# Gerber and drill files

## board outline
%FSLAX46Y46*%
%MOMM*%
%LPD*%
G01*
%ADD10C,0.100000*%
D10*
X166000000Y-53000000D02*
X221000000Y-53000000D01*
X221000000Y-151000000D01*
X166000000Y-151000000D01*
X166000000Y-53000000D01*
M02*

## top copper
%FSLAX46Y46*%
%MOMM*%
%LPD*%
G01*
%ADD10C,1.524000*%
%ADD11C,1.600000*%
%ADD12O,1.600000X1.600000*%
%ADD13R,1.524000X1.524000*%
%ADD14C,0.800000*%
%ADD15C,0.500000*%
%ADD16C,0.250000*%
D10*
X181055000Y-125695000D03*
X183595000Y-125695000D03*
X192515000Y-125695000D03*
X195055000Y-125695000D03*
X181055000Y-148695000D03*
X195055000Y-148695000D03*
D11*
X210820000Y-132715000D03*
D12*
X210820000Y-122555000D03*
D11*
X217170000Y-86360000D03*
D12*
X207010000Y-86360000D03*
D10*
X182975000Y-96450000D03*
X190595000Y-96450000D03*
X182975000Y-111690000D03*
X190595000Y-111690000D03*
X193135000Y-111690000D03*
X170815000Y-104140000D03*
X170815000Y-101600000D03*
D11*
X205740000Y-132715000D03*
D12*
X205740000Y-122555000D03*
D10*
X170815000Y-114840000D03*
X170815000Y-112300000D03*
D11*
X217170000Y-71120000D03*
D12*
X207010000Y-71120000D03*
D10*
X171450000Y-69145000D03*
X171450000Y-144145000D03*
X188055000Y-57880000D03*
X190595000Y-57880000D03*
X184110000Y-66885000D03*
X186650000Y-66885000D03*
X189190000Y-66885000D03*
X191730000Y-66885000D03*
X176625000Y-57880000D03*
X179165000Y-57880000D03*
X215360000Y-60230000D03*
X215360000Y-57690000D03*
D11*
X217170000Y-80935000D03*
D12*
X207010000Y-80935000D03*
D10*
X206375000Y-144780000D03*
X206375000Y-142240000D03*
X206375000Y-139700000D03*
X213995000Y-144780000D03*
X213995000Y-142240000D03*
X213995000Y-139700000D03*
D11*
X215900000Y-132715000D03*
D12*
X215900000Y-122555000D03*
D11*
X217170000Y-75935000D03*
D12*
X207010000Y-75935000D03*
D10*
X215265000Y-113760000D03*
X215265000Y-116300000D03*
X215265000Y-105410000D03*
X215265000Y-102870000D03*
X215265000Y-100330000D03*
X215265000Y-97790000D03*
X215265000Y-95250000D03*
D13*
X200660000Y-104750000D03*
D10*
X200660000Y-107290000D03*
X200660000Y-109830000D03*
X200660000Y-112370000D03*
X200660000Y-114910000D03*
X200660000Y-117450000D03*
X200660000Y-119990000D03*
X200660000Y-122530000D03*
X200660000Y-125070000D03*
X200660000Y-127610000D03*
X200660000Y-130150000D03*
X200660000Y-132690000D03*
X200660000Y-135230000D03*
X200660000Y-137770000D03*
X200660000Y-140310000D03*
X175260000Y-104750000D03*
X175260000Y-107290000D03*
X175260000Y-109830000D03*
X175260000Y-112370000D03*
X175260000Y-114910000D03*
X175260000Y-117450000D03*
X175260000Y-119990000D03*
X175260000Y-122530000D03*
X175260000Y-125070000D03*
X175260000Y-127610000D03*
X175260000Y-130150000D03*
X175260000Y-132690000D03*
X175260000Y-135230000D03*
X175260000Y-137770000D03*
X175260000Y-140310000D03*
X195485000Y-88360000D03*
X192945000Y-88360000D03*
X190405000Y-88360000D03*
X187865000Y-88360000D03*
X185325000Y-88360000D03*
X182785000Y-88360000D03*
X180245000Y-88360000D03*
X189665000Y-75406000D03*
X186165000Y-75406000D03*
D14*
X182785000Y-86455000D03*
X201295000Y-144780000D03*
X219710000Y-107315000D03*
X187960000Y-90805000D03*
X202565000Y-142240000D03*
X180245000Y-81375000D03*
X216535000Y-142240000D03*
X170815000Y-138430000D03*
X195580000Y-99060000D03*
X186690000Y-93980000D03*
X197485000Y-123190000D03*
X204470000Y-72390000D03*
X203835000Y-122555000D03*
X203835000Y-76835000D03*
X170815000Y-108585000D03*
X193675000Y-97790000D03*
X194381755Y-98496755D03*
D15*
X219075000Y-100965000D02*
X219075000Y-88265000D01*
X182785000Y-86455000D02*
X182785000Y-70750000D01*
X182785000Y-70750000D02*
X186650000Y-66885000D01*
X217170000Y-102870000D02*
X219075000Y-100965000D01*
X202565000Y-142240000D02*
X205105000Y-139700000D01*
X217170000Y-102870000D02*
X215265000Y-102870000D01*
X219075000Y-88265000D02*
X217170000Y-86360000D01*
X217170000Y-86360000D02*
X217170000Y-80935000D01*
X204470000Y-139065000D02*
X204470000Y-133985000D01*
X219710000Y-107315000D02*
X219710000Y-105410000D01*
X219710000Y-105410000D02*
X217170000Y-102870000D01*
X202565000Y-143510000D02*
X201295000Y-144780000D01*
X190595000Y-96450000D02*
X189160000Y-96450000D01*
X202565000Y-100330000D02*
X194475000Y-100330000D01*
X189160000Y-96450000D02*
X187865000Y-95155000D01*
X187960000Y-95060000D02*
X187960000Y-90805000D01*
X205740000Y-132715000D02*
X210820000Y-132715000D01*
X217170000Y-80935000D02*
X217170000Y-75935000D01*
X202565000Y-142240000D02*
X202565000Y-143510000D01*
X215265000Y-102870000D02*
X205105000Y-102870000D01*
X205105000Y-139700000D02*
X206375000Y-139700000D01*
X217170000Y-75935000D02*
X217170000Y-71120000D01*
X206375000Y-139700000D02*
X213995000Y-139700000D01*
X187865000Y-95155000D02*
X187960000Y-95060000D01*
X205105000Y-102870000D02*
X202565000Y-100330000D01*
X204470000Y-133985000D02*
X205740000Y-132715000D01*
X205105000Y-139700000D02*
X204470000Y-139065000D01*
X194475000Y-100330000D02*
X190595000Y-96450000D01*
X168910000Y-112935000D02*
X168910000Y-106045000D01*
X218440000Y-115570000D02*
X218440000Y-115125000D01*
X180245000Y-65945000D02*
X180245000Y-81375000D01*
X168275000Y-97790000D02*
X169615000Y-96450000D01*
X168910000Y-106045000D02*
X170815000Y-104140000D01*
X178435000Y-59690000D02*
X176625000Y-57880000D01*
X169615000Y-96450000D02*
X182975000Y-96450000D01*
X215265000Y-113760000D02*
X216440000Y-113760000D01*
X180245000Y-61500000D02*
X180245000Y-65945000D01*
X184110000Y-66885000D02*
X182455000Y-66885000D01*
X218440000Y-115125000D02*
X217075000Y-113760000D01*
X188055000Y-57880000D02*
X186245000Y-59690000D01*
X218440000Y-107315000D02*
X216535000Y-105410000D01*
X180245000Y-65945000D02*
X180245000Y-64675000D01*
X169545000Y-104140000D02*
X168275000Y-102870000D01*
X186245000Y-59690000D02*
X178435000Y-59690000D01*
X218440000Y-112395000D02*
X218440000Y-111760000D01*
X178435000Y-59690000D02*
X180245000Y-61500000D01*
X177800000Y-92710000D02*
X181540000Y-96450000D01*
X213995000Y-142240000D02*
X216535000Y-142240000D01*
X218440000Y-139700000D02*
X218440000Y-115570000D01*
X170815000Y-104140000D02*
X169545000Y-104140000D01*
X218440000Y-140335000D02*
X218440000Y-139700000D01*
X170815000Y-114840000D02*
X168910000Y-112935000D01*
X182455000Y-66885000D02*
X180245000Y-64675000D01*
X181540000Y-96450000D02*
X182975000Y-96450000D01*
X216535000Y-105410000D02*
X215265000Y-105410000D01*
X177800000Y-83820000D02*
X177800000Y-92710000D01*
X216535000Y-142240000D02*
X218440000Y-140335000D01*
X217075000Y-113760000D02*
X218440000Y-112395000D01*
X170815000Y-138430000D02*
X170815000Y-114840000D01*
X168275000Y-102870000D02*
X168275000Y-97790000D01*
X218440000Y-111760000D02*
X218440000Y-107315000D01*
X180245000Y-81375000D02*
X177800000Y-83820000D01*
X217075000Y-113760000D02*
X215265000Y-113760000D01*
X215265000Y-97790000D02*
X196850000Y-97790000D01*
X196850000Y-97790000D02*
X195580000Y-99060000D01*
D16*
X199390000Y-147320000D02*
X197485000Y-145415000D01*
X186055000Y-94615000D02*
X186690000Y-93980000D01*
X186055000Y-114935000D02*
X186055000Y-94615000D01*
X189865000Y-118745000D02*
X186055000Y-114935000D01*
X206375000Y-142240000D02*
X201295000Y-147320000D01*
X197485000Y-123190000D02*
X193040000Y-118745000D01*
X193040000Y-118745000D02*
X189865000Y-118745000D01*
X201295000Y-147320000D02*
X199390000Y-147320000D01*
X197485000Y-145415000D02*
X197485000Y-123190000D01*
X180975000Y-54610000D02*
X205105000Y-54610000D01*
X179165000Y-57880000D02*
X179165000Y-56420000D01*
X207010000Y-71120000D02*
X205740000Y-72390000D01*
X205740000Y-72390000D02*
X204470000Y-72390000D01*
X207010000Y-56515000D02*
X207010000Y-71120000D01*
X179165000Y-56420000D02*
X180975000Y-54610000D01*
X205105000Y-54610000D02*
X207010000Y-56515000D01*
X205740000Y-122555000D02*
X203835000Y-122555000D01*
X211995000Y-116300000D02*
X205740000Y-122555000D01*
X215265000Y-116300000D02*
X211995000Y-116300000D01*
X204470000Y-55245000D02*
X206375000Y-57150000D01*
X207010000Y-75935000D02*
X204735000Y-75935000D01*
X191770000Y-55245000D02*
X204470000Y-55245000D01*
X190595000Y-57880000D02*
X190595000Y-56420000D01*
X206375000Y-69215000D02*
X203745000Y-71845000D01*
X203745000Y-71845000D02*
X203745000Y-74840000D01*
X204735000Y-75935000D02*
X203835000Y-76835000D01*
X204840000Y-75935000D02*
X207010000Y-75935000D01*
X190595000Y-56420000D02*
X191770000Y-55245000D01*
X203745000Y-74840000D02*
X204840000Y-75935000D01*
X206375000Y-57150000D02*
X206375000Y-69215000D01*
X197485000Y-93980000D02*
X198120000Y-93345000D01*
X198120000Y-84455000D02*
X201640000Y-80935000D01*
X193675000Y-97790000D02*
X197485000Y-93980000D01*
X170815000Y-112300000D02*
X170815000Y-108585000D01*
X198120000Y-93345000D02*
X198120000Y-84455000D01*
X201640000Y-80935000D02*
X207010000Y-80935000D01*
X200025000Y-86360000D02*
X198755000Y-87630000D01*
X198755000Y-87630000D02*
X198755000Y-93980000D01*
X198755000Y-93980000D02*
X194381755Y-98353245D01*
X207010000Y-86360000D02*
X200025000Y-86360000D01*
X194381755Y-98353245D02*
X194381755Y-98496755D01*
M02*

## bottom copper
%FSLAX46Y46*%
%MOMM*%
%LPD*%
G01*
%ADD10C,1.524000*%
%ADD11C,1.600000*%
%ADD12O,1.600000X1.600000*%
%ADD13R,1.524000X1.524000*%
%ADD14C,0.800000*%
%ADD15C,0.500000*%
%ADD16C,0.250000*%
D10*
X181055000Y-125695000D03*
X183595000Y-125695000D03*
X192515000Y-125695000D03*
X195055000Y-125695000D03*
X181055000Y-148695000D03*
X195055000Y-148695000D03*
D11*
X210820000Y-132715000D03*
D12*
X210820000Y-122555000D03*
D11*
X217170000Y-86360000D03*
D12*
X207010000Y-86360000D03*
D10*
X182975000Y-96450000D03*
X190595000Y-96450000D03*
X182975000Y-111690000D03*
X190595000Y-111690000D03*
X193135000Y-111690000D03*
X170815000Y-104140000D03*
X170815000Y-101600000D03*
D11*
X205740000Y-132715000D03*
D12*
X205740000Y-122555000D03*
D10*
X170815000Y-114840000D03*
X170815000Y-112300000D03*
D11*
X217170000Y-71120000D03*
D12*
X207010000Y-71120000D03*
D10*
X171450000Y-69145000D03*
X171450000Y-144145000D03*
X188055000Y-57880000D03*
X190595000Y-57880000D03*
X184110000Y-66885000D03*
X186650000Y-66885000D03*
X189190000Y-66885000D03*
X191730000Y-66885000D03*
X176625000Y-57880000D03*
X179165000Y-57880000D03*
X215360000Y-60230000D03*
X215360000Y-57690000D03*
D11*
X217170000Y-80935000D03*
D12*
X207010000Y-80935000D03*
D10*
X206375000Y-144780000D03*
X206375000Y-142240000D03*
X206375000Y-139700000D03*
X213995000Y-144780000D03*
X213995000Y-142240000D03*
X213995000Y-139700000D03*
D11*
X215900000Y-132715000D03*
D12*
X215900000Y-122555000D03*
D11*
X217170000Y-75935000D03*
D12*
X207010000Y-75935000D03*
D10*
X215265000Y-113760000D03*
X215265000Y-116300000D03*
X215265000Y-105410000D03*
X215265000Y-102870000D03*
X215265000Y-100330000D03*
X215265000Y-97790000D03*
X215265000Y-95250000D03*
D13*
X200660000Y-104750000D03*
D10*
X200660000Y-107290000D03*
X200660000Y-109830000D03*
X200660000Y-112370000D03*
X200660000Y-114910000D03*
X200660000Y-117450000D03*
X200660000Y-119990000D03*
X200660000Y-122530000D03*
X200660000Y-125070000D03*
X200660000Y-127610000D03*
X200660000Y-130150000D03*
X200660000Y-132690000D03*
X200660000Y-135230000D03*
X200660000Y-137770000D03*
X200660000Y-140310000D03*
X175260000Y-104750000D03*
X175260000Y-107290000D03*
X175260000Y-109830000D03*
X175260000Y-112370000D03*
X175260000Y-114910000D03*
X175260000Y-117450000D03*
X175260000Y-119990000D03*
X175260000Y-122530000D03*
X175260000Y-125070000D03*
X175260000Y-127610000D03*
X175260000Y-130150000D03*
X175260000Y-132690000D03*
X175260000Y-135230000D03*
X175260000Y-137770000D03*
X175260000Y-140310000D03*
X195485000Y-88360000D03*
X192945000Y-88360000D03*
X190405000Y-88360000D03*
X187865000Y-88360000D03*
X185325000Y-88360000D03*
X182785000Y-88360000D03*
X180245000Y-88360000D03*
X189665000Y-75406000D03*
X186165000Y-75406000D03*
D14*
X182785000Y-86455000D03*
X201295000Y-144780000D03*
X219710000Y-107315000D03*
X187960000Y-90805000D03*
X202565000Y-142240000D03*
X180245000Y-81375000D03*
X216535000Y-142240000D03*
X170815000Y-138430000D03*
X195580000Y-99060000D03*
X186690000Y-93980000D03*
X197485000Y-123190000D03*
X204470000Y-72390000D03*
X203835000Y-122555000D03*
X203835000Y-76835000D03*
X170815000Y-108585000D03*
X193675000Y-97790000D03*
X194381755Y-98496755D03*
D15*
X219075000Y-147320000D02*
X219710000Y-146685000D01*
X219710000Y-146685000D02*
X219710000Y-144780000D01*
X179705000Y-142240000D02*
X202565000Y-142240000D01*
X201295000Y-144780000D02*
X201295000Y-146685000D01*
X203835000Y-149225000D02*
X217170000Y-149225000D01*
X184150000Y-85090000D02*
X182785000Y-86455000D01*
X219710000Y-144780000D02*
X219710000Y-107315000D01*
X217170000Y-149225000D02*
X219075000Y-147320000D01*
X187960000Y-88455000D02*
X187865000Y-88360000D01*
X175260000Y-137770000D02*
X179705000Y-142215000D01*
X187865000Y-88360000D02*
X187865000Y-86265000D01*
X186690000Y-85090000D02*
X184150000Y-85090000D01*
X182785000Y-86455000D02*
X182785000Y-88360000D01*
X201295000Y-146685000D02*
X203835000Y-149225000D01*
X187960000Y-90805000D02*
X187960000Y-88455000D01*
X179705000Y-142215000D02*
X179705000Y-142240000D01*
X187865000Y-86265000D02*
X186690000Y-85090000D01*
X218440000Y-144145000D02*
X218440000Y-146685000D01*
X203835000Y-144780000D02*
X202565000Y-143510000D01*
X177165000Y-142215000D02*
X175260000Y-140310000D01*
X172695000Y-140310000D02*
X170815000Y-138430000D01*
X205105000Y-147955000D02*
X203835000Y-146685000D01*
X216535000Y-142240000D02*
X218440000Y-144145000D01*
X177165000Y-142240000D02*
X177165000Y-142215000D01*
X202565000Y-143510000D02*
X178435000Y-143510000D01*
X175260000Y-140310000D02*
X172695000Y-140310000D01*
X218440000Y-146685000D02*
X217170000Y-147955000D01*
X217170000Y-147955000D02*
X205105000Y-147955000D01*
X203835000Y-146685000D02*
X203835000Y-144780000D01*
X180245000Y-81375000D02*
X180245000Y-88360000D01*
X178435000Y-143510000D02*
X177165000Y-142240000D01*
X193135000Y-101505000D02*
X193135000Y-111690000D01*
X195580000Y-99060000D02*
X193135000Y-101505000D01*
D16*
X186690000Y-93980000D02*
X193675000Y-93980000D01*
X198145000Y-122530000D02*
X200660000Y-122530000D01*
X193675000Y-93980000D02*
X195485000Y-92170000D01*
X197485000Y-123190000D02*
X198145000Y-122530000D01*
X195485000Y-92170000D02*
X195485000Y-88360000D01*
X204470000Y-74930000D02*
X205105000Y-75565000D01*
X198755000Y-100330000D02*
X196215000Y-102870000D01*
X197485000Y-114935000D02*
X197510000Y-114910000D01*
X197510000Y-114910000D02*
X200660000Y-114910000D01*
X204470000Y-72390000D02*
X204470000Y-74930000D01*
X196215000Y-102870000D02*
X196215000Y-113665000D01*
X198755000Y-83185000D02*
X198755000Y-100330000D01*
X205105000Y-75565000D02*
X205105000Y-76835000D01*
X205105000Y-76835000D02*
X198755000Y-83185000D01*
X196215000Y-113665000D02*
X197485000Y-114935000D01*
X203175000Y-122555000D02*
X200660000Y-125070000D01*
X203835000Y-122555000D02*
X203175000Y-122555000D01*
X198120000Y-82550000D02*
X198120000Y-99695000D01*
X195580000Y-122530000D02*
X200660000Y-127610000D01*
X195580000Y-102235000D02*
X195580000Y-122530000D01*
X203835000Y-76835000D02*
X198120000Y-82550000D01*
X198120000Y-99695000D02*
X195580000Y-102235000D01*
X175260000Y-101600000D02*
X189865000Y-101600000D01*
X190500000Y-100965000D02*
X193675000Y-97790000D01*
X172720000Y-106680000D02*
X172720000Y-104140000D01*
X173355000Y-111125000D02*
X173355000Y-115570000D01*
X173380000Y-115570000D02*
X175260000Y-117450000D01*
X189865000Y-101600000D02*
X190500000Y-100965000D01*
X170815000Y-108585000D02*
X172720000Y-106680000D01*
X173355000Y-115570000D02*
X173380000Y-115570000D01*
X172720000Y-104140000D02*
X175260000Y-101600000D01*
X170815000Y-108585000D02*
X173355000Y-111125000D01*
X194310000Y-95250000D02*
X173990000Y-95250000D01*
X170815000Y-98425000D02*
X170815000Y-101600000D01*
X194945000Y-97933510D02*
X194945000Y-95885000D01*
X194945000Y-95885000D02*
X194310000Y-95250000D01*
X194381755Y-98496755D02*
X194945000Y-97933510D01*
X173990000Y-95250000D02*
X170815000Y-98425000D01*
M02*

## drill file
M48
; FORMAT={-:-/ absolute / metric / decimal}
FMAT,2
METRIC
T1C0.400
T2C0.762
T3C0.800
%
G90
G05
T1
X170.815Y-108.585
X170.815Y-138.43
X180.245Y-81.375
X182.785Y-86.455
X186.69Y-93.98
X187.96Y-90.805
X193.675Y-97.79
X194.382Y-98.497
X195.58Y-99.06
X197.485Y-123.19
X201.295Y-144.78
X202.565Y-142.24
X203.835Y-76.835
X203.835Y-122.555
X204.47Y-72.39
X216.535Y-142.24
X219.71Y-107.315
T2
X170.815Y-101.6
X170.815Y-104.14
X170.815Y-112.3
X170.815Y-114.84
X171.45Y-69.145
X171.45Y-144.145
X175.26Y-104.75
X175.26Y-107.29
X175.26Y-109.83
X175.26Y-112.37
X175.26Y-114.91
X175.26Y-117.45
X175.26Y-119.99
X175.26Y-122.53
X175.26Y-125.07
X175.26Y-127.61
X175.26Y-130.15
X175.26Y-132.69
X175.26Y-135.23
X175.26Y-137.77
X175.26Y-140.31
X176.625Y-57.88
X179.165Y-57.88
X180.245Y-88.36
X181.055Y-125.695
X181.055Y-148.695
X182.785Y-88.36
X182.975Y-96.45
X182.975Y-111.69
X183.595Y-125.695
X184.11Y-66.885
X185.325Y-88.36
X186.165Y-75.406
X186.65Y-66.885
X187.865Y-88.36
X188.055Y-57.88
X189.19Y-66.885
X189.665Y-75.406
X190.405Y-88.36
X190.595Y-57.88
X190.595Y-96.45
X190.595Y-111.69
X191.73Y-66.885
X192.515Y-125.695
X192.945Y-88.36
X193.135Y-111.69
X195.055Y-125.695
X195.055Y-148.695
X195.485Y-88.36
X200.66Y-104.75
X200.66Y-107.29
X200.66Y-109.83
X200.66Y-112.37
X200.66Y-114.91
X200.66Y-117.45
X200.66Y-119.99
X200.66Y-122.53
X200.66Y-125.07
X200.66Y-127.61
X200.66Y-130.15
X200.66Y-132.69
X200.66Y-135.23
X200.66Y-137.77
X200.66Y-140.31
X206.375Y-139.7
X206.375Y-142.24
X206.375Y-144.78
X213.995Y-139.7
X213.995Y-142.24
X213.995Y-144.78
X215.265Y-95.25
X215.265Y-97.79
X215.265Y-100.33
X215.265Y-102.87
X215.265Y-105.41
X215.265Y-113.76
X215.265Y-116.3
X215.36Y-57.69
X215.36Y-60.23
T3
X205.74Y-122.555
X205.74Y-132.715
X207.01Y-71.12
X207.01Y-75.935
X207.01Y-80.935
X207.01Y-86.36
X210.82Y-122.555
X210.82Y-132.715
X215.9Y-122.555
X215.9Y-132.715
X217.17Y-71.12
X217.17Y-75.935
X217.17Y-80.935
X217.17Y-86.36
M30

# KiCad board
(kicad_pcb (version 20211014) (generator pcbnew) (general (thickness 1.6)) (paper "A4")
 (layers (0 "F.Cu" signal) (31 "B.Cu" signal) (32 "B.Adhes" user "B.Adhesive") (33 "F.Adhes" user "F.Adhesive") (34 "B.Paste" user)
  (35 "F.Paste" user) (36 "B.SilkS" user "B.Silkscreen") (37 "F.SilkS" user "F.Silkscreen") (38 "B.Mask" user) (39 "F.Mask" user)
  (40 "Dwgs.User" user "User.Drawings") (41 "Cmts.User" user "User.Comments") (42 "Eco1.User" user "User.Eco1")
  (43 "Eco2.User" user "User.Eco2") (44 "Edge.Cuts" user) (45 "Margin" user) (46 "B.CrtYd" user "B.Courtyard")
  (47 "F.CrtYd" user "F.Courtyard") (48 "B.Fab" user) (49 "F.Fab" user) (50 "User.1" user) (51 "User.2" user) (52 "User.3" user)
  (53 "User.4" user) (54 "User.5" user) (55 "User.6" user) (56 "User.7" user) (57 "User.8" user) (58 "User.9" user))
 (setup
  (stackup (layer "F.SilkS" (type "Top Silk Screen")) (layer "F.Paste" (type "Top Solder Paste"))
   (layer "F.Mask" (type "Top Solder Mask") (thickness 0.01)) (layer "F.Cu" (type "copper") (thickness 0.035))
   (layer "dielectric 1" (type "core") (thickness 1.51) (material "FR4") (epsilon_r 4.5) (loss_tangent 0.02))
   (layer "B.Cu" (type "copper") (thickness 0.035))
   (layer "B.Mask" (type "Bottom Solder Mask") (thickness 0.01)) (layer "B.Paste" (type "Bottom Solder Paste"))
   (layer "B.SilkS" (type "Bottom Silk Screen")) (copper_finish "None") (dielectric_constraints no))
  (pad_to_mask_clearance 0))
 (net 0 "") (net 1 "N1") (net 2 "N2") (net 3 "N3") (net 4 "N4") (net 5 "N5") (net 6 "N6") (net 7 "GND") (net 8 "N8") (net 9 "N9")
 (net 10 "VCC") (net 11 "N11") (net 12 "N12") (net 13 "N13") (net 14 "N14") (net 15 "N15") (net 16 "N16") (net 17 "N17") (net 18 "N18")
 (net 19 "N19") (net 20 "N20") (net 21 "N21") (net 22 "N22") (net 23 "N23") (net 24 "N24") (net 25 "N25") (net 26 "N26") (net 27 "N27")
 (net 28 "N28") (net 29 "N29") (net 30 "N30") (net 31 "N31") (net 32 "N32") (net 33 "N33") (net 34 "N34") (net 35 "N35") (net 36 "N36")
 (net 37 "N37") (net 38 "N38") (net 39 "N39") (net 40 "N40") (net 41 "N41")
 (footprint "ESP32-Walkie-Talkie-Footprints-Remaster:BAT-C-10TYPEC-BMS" (layer "F.Cu") (at 179.455 123.255)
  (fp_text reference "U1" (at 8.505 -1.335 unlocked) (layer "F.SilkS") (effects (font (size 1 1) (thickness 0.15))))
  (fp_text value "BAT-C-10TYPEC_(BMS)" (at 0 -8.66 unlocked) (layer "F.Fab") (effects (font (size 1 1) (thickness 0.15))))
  (pad "1" thru_hole circle (at 1.6 2.44) (size 1.524 1.524) (drill 0.762) (layers *.Cu *.Mask) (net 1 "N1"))
  (pad "2" thru_hole circle (at 4.14 2.44) (size 1.524 1.524) (drill 0.762) (layers *.Cu *.Mask) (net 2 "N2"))
  (pad "3" thru_hole circle (at 13.06 2.44) (size 1.524 1.524) (drill 0.762) (layers *.Cu *.Mask) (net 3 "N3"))
  (pad "4" thru_hole circle (at 15.6 2.44) (size 1.524 1.524) (drill 0.762) (layers *.Cu *.Mask) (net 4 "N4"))
  (pad "5" thru_hole circle (at 1.6 25.44) (size 1.524 1.524) (drill 0.762) (layers *.Cu *.Mask) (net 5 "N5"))
  (pad "6" thru_hole circle (at 15.6 25.44) (size 1.524 1.524) (drill 0.762) (layers *.Cu *.Mask) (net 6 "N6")))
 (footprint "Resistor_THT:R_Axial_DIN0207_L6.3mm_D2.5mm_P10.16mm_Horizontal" (layer "F.Cu") (at 210.82 132.715 90)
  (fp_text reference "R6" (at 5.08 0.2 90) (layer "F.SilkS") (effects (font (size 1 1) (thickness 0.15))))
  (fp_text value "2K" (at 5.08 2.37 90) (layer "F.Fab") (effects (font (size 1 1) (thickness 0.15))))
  (pad "1" thru_hole circle (at 0 0 90) (size 1.6 1.6) (drill 0.8) (layers *.Cu *.Mask) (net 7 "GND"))
  (pad "2" thru_hole oval (at 10.16 0 90) (size 1.6 1.6) (drill 0.8) (layers *.Cu *.Mask) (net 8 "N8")))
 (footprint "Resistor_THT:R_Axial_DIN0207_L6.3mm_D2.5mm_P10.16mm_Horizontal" (layer "F.Cu") (at 217.17 86.36 180)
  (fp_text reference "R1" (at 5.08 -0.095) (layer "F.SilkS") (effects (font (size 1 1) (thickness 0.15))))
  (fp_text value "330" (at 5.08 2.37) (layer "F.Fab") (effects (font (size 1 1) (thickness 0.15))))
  (pad "1" thru_hole circle (at 0 0 180) (size 1.6 1.6) (drill 0.8) (layers *.Cu *.Mask) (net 7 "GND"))
  (pad "2" thru_hole oval (at 10.16 0 180) (size 1.6 1.6) (drill 0.8) (layers *.Cu *.Mask) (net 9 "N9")))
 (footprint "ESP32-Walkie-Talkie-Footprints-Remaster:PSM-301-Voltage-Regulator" (layer "F.Cu") (at 181.03 94.835)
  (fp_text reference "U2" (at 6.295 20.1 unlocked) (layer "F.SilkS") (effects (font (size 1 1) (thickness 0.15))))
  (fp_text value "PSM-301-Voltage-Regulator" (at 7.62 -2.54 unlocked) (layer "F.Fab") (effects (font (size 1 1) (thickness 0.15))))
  (pad "1" thru_hole circle (at 1.945 1.615) (size 1.524 1.524) (drill 0.762) (layers *.Cu *.Mask) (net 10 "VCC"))
  (pad "2" thru_hole circle (at 9.565 1.615) (size 1.524 1.524) (drill 0.762) (layers *.Cu *.Mask) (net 7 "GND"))
  (pad "3" thru_hole circle (at 1.945 16.855) (size 1.524 1.524) (drill 0.762) (layers *.Cu *.Mask) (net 4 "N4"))
  (pad "4" thru_hole circle (at 9.565 16.855) (size 1.524 1.524) (drill 0.762) (layers *.Cu *.Mask) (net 1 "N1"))
  (pad "5" thru_hole circle (at 12.105 16.855) (size 1.524 1.524) (drill 0.762) (layers *.Cu *.Mask) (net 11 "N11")))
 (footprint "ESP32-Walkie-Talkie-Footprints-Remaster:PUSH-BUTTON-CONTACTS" (layer "F.Cu") (at 168.275 106.68 90)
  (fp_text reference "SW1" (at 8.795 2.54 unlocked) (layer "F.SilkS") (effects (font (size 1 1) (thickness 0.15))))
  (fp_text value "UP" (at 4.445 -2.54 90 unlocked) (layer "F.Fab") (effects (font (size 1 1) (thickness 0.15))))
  (pad "1" thru_hole circle (at 2.54 2.54 90) (size 1.524 1.524) (drill 0.762) (layers *.Cu *.Mask) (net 10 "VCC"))
  (pad "2" thru_hole circle (at 5.08 2.54 90) (size 1.524 1.524) (drill 0.762) (layers *.Cu *.Mask) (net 9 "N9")))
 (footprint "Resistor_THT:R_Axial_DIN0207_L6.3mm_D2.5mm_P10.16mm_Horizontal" (layer "F.Cu") (at 205.74 132.715 90)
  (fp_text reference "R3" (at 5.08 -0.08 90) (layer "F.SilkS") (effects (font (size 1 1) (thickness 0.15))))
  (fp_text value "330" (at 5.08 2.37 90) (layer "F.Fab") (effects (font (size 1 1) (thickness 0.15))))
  (pad "1" thru_hole circle (at 0 0 90) (size 1.6 1.6) (drill 0.8) (layers *.Cu *.Mask) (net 7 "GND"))
  (pad "2" thru_hole oval (at 10.16 0 90) (size 1.6 1.6) (drill 0.8) (layers *.Cu *.Mask) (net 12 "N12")))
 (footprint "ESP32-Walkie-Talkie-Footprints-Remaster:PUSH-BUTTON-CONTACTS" (layer "F.Cu") (at 168.275 117.38 90)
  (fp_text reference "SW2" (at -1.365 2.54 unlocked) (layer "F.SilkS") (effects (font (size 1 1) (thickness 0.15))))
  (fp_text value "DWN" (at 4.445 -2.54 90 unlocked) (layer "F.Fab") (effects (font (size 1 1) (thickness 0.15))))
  (pad "1" thru_hole circle (at 2.54 2.54 90) (size 1.524 1.524) (drill 0.762) (layers *.Cu *.Mask) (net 10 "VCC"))
  (pad "2" thru_hole circle (at 5.08 2.54 90) (size 1.524 1.524) (drill 0.762) (layers *.Cu *.Mask) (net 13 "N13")))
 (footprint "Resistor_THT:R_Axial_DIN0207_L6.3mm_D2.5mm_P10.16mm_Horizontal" (layer "F.Cu") (at 217.17 71.12 180)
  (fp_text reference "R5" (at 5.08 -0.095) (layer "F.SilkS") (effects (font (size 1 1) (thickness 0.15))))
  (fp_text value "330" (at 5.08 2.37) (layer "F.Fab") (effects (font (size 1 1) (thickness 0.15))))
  (pad "1" thru_hole circle (at 0 0 180) (size 1.6 1.6) (drill 0.8) (layers *.Cu *.Mask) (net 7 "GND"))
  (pad "2" thru_hole oval (at 10.16 0 180) (size 1.6 1.6) (drill 0.8) (layers *.Cu *.Mask) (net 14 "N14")))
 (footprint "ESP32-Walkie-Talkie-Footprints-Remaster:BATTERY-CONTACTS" (layer "F.Cu") (at 171.45 69.145)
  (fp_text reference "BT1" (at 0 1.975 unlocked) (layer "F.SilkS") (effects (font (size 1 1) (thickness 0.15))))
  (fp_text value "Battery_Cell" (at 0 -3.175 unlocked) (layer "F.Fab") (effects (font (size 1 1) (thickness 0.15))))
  (pad "1" thru_hole circle (at 0 0) (size 1.524 1.524) (drill 0.762) (layers *.Cu *.Mask) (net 2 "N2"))
  (pad "2" thru_hole circle (at 0 75) (size 1.524 1.524) (drill 0.762) (layers *.Cu *.Mask) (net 3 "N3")))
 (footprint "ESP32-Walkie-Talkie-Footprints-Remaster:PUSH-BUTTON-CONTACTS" (layer "F.Cu") (at 185.515 55.34)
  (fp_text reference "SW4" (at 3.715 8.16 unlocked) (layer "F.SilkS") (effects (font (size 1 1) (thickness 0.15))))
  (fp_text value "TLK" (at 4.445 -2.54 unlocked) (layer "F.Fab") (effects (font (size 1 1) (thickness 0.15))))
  (pad "1" thru_hole circle (at 2.54 2.54) (size 1.524 1.524) (drill 0.762) (layers *.Cu *.Mask) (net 10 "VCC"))
  (pad "2" thru_hole circle (at 5.08 2.54) (size 1.524 1.524) (drill 0.762) (layers *.Cu *.Mask) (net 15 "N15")))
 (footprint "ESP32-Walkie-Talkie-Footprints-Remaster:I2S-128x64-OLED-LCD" (layer "F.Cu") (at 188.91 65.185)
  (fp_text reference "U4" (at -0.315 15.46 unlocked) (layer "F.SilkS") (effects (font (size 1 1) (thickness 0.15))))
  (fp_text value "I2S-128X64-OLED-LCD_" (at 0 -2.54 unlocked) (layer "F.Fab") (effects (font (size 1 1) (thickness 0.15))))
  (pad "1" thru_hole circle (at -4.8 1.7) (size 1.524 1.524) (drill 0.762) (layers *.Cu *.Mask) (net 10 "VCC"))
  (pad "2" thru_hole circle (at -2.26 1.7) (size 1.524 1.524) (drill 0.762) (layers *.Cu *.Mask) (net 7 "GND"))
  (pad "3" thru_hole circle (at 0.28 1.7) (size 1.524 1.524) (drill 0.762) (layers *.Cu *.Mask) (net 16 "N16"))
  (pad "4" thru_hole circle (at 2.82 1.7) (size 1.524 1.524) (drill 0.762) (layers *.Cu *.Mask) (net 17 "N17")))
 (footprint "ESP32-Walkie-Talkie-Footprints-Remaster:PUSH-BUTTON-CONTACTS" (layer "F.Cu") (at 174.085 55.34)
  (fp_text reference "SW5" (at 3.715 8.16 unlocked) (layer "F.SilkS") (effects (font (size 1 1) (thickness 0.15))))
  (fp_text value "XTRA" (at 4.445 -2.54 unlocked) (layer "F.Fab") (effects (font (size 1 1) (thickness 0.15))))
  (pad "1" thru_hole circle (at 2.54 2.54) (size 1.524 1.524) (drill 0.762) (layers *.Cu *.Mask) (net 10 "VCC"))
  (pad "2" thru_hole circle (at 5.08 2.54) (size 1.524 1.524) (drill 0.762) (layers *.Cu *.Mask) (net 14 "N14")))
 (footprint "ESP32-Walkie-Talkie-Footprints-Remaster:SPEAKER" (layer "F.Cu") (at 212.82 62.77 90)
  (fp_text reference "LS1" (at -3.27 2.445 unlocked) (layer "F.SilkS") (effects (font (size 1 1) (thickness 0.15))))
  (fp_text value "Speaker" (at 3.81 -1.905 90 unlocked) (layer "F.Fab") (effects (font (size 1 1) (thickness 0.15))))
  (pad "1" thru_hole circle (at 2.54 2.54 90) (size 1.524 1.524) (drill 0.762) (layers *.Cu *.Mask) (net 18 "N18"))
  (pad "2" thru_hole circle (at 5.08 2.54 90) (size 1.524 1.524) (drill 0.762) (layers *.Cu *.Mask) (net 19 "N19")))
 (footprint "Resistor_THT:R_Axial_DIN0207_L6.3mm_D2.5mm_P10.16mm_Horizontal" (layer "F.Cu") (at 217.17 80.935 180)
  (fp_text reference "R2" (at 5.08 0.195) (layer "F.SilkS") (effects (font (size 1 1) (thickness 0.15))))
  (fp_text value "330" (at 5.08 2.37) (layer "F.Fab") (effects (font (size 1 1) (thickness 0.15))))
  (pad "1" thru_hole circle (at 0 0 180) (size 1.6 1.6) (drill 0.8) (layers *.Cu *.Mask) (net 7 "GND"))
  (pad "2" thru_hole oval (at 10.16 0 180) (size 1.6 1.6) (drill 0.8) (layers *.Cu *.Mask) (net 13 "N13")))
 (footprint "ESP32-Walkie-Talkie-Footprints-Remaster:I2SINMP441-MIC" (layer "F.Cu") (at 208.915 142.24 90)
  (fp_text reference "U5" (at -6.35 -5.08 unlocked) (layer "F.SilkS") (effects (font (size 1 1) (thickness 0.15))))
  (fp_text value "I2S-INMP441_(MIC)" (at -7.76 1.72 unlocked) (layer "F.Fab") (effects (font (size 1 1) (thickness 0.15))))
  (pad "1" thru_hole circle (at -2.54 -2.54 90) (size 1.524 1.524) (drill 0.762) (layers *.Cu *.Mask) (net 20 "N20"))
  (pad "2" thru_hole circle (at 0 -2.54 90) (size 1.524 1.524) (drill 0.762) (layers *.Cu *.Mask) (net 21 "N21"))
  (pad "3" thru_hole circle (at 2.54 -2.54 90) (size 1.524 1.524) (drill 0.762) (layers *.Cu *.Mask) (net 7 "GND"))
  (pad "4" thru_hole circle (at -2.54 5.08 90) (size 1.524 1.524) (drill 0.762) (layers *.Cu *.Mask) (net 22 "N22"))
  (pad "5" thru_hole circle (at 0 5.08 90) (size 1.524 1.524) (drill 0.762) (layers *.Cu *.Mask) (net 10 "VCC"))
  (pad "6" thru_hole circle (at 2.54 5.08 90) (size 1.524 1.524) (drill 0.762) (layers *.Cu *.Mask) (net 7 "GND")))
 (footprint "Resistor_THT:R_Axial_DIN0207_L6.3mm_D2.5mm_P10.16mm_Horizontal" (layer "F.Cu") (at 215.9 132.715 90)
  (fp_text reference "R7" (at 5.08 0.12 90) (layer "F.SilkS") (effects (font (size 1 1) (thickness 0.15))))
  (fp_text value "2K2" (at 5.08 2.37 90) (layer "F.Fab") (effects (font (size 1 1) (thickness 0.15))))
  (pad "1" thru_hole circle (at 0 0 90) (size 1.6 1.6) (drill 0.8) (layers *.Cu *.Mask) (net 8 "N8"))
  (pad "2" thru_hole oval (at 10.16 0 90) (size 1.6 1.6) (drill 0.8) (layers *.Cu *.Mask) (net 2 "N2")))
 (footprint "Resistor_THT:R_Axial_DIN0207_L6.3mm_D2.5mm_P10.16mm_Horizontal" (layer "F.Cu") (at 217.17 75.935 180)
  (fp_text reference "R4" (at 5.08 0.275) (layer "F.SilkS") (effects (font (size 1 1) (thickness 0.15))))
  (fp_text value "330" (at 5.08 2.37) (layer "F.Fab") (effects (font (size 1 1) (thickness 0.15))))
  (pad "1" thru_hole circle (at 0 0 180) (size 1.6 1.6) (drill 0.8) (layers *.Cu *.Mask) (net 7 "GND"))
  (pad "2" thru_hole oval (at 10.16 0 180) (size 1.6 1.6) (drill 0.8) (layers *.Cu *.Mask) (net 15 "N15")))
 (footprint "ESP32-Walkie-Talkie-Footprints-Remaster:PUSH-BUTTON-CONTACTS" (layer "F.Cu") (at 217.805 111.22 -90)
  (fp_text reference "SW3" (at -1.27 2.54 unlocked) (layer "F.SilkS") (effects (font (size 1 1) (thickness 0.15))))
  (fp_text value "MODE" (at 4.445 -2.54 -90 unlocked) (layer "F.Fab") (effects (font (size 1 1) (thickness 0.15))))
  (pad "1" thru_hole circle (at 2.54 2.54 270) (size 1.524 1.524) (drill 0.762) (layers *.Cu *.Mask) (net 10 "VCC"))
  (pad "2" thru_hole circle (at 5.08 2.54 270) (size 1.524 1.524) (drill 0.762) (layers *.Cu *.Mask) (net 12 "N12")))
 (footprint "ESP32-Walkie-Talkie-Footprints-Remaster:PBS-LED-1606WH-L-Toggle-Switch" (layer "F.Cu") (at 212.725 107.95 90)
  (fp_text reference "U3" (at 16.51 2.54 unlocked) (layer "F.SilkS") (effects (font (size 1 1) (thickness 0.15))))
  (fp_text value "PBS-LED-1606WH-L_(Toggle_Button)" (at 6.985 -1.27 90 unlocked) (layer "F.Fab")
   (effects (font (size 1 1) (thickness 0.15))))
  (pad "1" thru_hole circle (at 2.54 2.54 90) (size 1.524 1.524) (drill 0.762) (layers *.Cu *.Mask) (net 10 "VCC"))
  (pad "2" thru_hole circle (at 5.08 2.54 90) (size 1.524 1.524) (drill 0.762) (layers *.Cu *.Mask) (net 7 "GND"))
  (pad "3" thru_hole circle (at 7.62 2.54 90) (size 1.524 1.524) (drill 0.762) (layers *.Cu *.Mask) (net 2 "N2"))
  (pad "4" thru_hole circle (at 10.16 2.54 90) (size 1.524 1.524) (drill 0.762) (layers *.Cu *.Mask) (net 11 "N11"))
  (pad "5" thru_hole circle (at 12.7 2.54 90) (size 1.524 1.524) (drill 0.762) (layers *.Cu *.Mask) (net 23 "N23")))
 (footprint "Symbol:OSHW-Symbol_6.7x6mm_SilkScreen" (layer "B.Cu") (at 170.815 57.15 180)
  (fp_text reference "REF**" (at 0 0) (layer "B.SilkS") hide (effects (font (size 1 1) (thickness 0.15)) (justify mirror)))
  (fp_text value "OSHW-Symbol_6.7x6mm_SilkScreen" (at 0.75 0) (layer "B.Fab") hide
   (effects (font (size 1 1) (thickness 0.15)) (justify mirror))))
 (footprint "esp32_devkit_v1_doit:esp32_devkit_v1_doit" (layer "B.Cu") (at 187.96 104.75 180)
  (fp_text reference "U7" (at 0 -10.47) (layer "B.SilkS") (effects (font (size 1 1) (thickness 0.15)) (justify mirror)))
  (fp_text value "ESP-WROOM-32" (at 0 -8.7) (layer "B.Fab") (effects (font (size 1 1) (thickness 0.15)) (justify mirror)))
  (pad "1" thru_hole rect (at -12.7 0 180) (size 1.524 1.524) (drill 0.762) (layers *.Cu *.Mask) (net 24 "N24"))
  (pad "2" thru_hole circle (at -12.7 -2.54 180) (size 1.524 1.524) (drill 0.762) (layers *.Cu *.Mask) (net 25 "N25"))
  (pad "3" thru_hole circle (at -12.7 -5.08 180) (size 1.524 1.524) (drill 0.762) (layers *.Cu *.Mask) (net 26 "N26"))
  (pad "4" thru_hole circle (at -12.7 -7.62 180) (size 1.524 1.524) (drill 0.762) (layers *.Cu *.Mask) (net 8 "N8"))
  (pad "5" thru_hole circle (at -12.7 -10.16 180) (size 1.524 1.524) (drill 0.762) (layers *.Cu *.Mask) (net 14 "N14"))
  (pad "6" thru_hole circle (at -12.7 -12.7 180) (size 1.524 1.524) (drill 0.762) (layers *.Cu *.Mask) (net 20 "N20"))
  (pad "7" thru_hole circle (at -12.7 -15.24 180) (size 1.524 1.524) (drill 0.762) (layers *.Cu *.Mask) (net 22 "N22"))
  (pad "8" thru_hole circle (at -12.7 -17.78 180) (size 1.524 1.524) (drill 0.762) (layers *.Cu *.Mask) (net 21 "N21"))
  (pad "9" thru_hole circle (at -12.7 -20.32 180) (size 1.524 1.524) (drill 0.762) (layers *.Cu *.Mask) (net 12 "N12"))
  (pad "10" thru_hole circle (at -12.7 -22.86 180) (size 1.524 1.524) (drill 0.762) (layers *.Cu *.Mask) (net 15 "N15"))
  (pad "11" thru_hole circle (at -12.7 -25.4 180) (size 1.524 1.524) (drill 0.762) (layers *.Cu *.Mask) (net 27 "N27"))
  (pad "12" thru_hole circle (at -12.7 -27.94 180) (size 1.524 1.524) (drill 0.762) (layers *.Cu *.Mask) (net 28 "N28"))
  (pad "13" thru_hole circle (at -12.7 -30.48 180) (size 1.524 1.524) (drill 0.762) (layers *.Cu *.Mask) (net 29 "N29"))
  (pad "14" thru_hole circle (at -12.7 -33.02 180) (size 1.524 1.524) (drill 0.762) (layers *.Cu *.Mask) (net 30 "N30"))
  (pad "15" thru_hole circle (at -12.7 -35.56 180) (size 1.524 1.524) (drill 0.762) (layers *.Cu *.Mask) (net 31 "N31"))
  (pad "16" thru_hole circle (at 12.7 0 180) (size 1.524 1.524) (drill 0.762) (layers *.Cu *.Mask) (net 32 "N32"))
  (pad "17" thru_hole circle (at 12.7 -2.54 180) (size 1.524 1.524) (drill 0.762) (layers *.Cu *.Mask) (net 16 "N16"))
  (pad "18" thru_hole circle (at 12.7 -5.08 180) (size 1.524 1.524) (drill 0.762) (layers *.Cu *.Mask) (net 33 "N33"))
  (pad "19" thru_hole circle (at 12.7 -7.62 180) (size 1.524 1.524) (drill 0.762) (layers *.Cu *.Mask) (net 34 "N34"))
  (pad "20" thru_hole circle (at 12.7 -10.16 180) (size 1.524 1.524) (drill 0.762) (layers *.Cu *.Mask) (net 17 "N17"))
  (pad "21" thru_hole circle (at 12.7 -12.7 180) (size 1.524 1.524) (drill 0.762) (layers *.Cu *.Mask) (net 13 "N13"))
  (pad "22" thru_hole circle (at 12.7 -15.24 180) (size 1.524 1.524) (drill 0.762) (layers *.Cu *.Mask) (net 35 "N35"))
  (pad "23" thru_hole circle (at 12.7 -17.78 180) (size 1.524 1.524) (drill 0.762) (layers *.Cu *.Mask) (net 9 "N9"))
  (pad "24" thru_hole circle (at 12.7 -20.32 180) (size 1.524 1.524) (drill 0.762) (layers *.Cu *.Mask) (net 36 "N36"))
  (pad "25" thru_hole circle (at 12.7 -22.86 180) (size 1.524 1.524) (drill 0.762) (layers *.Cu *.Mask) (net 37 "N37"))
  (pad "26" thru_hole circle (at 12.7 -25.4 180) (size 1.524 1.524) (drill 0.762) (layers *.Cu *.Mask) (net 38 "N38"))
  (pad "27" thru_hole circle (at 12.7 -27.94 180) (size 1.524 1.524) (drill 0.762) (layers *.Cu *.Mask) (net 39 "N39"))
  (pad "28" thru_hole circle (at 12.7 -30.48 180) (size 1.524 1.524) (drill 0.762) (layers *.Cu *.Mask) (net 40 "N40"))
  (pad "29" thru_hole circle (at 12.7 -33.02 180) (size 1.524 1.524) (drill 0.762) (layers *.Cu *.Mask) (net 7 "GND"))
  (pad "30" thru_hole circle (at 12.7 -35.56 180) (size 1.524 1.524) (drill 0.762) (layers *.Cu *.Mask) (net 10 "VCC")))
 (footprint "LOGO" (layer "B.Cu") (at 203.2 60.325 180)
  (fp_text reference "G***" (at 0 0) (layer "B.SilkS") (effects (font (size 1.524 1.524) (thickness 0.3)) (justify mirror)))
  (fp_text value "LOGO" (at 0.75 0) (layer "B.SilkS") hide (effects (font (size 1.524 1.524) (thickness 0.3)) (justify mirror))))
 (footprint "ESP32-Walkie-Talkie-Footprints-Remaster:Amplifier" (layer "B.Cu") (at 196.755 71.85 180)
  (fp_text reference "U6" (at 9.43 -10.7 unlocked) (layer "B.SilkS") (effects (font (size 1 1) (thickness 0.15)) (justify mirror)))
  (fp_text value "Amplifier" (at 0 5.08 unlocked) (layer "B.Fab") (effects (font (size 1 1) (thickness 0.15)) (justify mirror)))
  (pad "1" thru_hole circle (at 1.27 -16.51 180) (size 1.524 1.524) (drill 0.762) (layers *.Cu *.Mask) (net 21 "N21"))
  (pad "2" thru_hole circle (at 3.81 -16.51 180) (size 1.524 1.524) (drill 0.762) (layers *.Cu *.Mask) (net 20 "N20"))
  (pad "3" thru_hole circle (at 6.35 -16.51 180) (size 1.524 1.524) (drill 0.762) (layers *.Cu *.Mask) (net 27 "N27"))
  (pad "4" thru_hole circle (at 8.89 -16.51 180) (size 1.524 1.524) (drill 0.762) (layers *.Cu *.Mask) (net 7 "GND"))
  (pad "5" thru_hole circle (at 11.43 -16.51 180) (size 1.524 1.524) (drill 0.762) (layers *.Cu *.Mask) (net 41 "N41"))
  (pad "6" thru_hole circle (at 13.97 -16.51 180) (size 1.524 1.524) (drill 0.762) (layers *.Cu *.Mask) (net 7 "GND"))
  (pad "7" thru_hole circle (at 16.51 -16.51 180) (size 1.524 1.524) (drill 0.762) (layers *.Cu *.Mask) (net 10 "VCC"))
  (pad "8" thru_hole circle (at 7.09 -3.556 180) (size 1.524 1.524) (drill 0.762) (layers *.Cu *.Mask) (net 18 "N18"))
  (pad "9" thru_hole circle (at 10.59 -3.556 180) (size 1.524 1.524) (drill 0.762) (layers *.Cu *.Mask) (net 19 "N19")))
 (gr_rect (start 166 53) (end 221 151) (layer "Edge.Cuts") (width 0.1) (fill none))
 (segment (start 219.075 100.965) (end 219.075 88.265) (width 0.5) (layer "F.Cu") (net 7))
 (segment (start 182.785 86.455) (end 182.785 70.75) (width 0.5) (layer "F.Cu") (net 7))
 (segment (start 182.785 70.75) (end 186.65 66.885) (width 0.5) (layer "F.Cu") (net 7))
 (segment (start 217.17 102.87) (end 219.075 100.965) (width 0.5) (layer "F.Cu") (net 7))
 (segment (start 202.565 142.24) (end 205.105 139.7) (width 0.5) (layer "F.Cu") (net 7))
 (segment (start 217.17 102.87) (end 215.265 102.87) (width 0.5) (layer "F.Cu") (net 7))
 (segment (start 219.075 88.265) (end 217.17 86.36) (width 0.5) (layer "F.Cu") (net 7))
 (segment (start 217.17 86.36) (end 217.17 80.935) (width 0.5) (layer "F.Cu") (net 7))
 (segment (start 204.47 139.065) (end 204.47 133.985) (width 0.5) (layer "F.Cu") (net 7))
 (segment (start 219.71 107.315) (end 219.71 105.41) (width 0.5) (layer "F.Cu") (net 7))
 (segment (start 219.71 105.41) (end 217.17 102.87) (width 0.5) (layer "F.Cu") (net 7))
 (segment (start 202.565 143.51) (end 201.295 144.78) (width 0.5) (layer "F.Cu") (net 7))
 (segment (start 190.595 96.45) (end 189.16 96.45) (width 0.5) (layer "F.Cu") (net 7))
 (segment (start 202.565 100.33) (end 194.475 100.33) (width 0.5) (layer "F.Cu") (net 7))
 (segment (start 189.16 96.45) (end 187.865 95.155) (width 0.5) (layer "F.Cu") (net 7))
 (segment (start 187.96 95.06) (end 187.96 90.805) (width 0.5) (layer "F.Cu") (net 7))
 (segment (start 205.74 132.715) (end 210.82 132.715) (width 0.5) (layer "F.Cu") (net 7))
 (segment (start 217.17 80.935) (end 217.17 75.935) (width 0.5) (layer "F.Cu") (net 7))
 (segment (start 202.565 142.24) (end 202.565 143.51) (width 0.5) (layer "F.Cu") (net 7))
 (segment (start 215.265 102.87) (end 205.105 102.87) (width 0.5) (layer "F.Cu") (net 7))
 (segment (start 205.105 139.7) (end 206.375 139.7) (width 0.5) (layer "F.Cu") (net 7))
 (segment (start 217.17 75.935) (end 217.17 71.12) (width 0.5) (layer "F.Cu") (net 7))
 (segment (start 206.375 139.7) (end 213.995 139.7) (width 0.5) (layer "F.Cu") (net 7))
 (segment (start 187.865 95.155) (end 187.96 95.06) (width 0.5) (layer "F.Cu") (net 7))
 (segment (start 205.105 102.87) (end 202.565 100.33) (width 0.5) (layer "F.Cu") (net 7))
 (segment (start 204.47 133.985) (end 205.74 132.715) (width 0.5) (layer "F.Cu") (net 7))
 (segment (start 205.105 139.7) (end 204.47 139.065) (width 0.5) (layer "F.Cu") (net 7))
 (segment (start 194.475 100.33) (end 190.595 96.45) (width 0.5) (layer "F.Cu") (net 7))
 (via (at 182.785 86.455) (size 0.8) (drill 0.4) (layers "F.Cu" "B.Cu") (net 7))
 (via (at 201.295 144.78) (size 0.8) (drill 0.4) (layers "F.Cu" "B.Cu") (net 7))
 (via (at 219.71 107.315) (size 0.8) (drill 0.4) (layers "F.Cu" "B.Cu") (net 7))
 (via (at 187.96 90.805) (size 0.8) (drill 0.4) (layers "F.Cu" "B.Cu") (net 7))
 (via (at 202.565 142.24) (size 0.8) (drill 0.4) (layers "F.Cu" "B.Cu") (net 7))
 (segment (start 219.075 147.32) (end 219.71 146.685) (width 0.5) (layer "B.Cu") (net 7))
 (segment (start 219.71 146.685) (end 219.71 144.78) (width 0.5) (layer "B.Cu") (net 7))
 (segment (start 179.705 142.24) (end 202.565 142.24) (width 0.5) (layer "B.Cu") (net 7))
 (segment (start 201.295 144.78) (end 201.295 146.685) (width 0.5) (layer "B.Cu") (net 7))
 (segment (start 203.835 149.225) (end 217.17 149.225) (width 0.5) (layer "B.Cu") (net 7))
 (segment (start 184.15 85.09) (end 182.785 86.455) (width 0.5) (layer "B.Cu") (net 7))
 (segment (start 219.71 144.78) (end 219.71 107.315) (width 0.5) (layer "B.Cu") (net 7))
 (segment (start 217.17 149.225) (end 219.075 147.32) (width 0.5) (layer "B.Cu") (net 7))
 (segment (start 187.96 88.455) (end 187.865 88.36) (width 0.5) (layer "B.Cu") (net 7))
 (segment (start 175.26 137.77) (end 179.705 142.215) (width 0.5) (layer "B.Cu") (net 7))
 (segment (start 187.865 88.36) (end 187.865 86.265) (width 0.5) (layer "B.Cu") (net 7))
 (segment (start 186.69 85.09) (end 184.15 85.09) (width 0.5) (layer "B.Cu") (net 7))
 (segment (start 182.785 86.455) (end 182.785 88.36) (width 0.5) (layer "B.Cu") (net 7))
 (segment (start 201.295 146.685) (end 203.835 149.225) (width 0.5) (layer "B.Cu") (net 7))
 (segment (start 187.96 90.805) (end 187.96 88.455) (width 0.5) (layer "B.Cu") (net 7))
 (segment (start 179.705 142.215) (end 179.705 142.24) (width 0.5) (layer "B.Cu") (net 7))
 (segment (start 187.865 86.265) (end 186.69 85.09) (width 0.5) (layer "B.Cu") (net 7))
 (segment (start 168.91 112.935) (end 168.91 106.045) (width 0.5) (layer "F.Cu") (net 10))
 (segment (start 218.44 115.57) (end 218.44 115.125) (width 0.5) (layer "F.Cu") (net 10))
 (segment (start 180.245 65.945) (end 180.245 81.375) (width 0.5) (layer "F.Cu") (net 10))
 (segment (start 168.275 97.79) (end 169.615 96.45) (width 0.5) (layer "F.Cu") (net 10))
 (segment (start 168.91 106.045) (end 170.815 104.14) (width 0.5) (layer "F.Cu") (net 10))
 (segment (start 178.435 59.69) (end 176.625 57.88) (width 0.5) (layer "F.Cu") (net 10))
 (segment (start 169.615 96.45) (end 182.975 96.45) (width 0.5) (layer "F.Cu") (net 10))
 (segment (start 215.265 113.76) (end 216.44 113.76) (width 0.5) (layer "F.Cu") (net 10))
 (segment (start 180.245 61.5) (end 180.245 65.945) (width 0.5) (layer "F.Cu") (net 10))
 (segment (start 184.11 66.885) (end 182.455 66.885) (width 0.5) (layer "F.Cu") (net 10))
 (segment (start 218.44 115.125) (end 217.075 113.76) (width 0.5) (layer "F.Cu") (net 10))
 (segment (start 188.055 57.88) (end 186.245 59.69) (width 0.5) (layer "F.Cu") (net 10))
 (segment (start 218.44 107.315) (end 216.535 105.41) (width 0.5) (layer "F.Cu") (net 10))
 (segment (start 180.245 65.945) (end 180.245 64.675) (width 0.5) (layer "F.Cu") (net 10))
 (segment (start 169.545 104.14) (end 168.275 102.87) (width 0.5) (layer "F.Cu") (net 10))
 (segment (start 186.245 59.69) (end 178.435 59.69) (width 0.5) (layer "F.Cu") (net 10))
 (segment (start 218.44 112.395) (end 218.44 111.76) (width 0.5) (layer "F.Cu") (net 10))
 (segment (start 178.435 59.69) (end 180.245 61.5) (width 0.5) (layer "F.Cu") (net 10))
 (segment (start 177.8 92.71) (end 181.54 96.45) (width 0.5) (layer "F.Cu") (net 10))
 (segment (start 213.995 142.24) (end 216.535 142.24) (width 0.5) (layer "F.Cu") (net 10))
 (segment (start 218.44 139.7) (end 218.44 115.57) (width 0.5) (layer "F.Cu") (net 10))
 (segment (start 170.815 104.14) (end 169.545 104.14) (width 0.5) (layer "F.Cu") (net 10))
 (segment (start 218.44 140.335) (end 218.44 139.7) (width 0.5) (layer "F.Cu") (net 10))
 (segment (start 170.815 114.84) (end 168.91 112.935) (width 0.5) (layer "F.Cu") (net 10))
 (segment (start 182.455 66.885) (end 180.245 64.675) (width 0.5) (layer "F.Cu") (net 10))
 (segment (start 181.54 96.45) (end 182.975 96.45) (width 0.5) (layer "F.Cu") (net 10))
 (segment (start 216.535 105.41) (end 215.265 105.41) (width 0.5) (layer "F.Cu") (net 10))
 (segment (start 177.8 83.82) (end 177.8 92.71) (width 0.5) (layer "F.Cu") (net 10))
 (segment (start 216.535 142.24) (end 218.44 140.335) (width 0.5) (layer "F.Cu") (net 10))
 (segment (start 217.075 113.76) (end 218.44 112.395) (width 0.5) (layer "F.Cu") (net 10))
 (segment (start 170.815 138.43) (end 170.815 114.84) (width 0.5) (layer "F.Cu") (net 10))
 (segment (start 168.275 102.87) (end 168.275 97.79) (width 0.5) (layer "F.Cu") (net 10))
 (segment (start 218.44 111.76) (end 218.44 107.315) (width 0.5) (layer "F.Cu") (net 10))
 (segment (start 180.245 81.375) (end 177.8 83.82) (width 0.5) (layer "F.Cu") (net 10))
 (segment (start 217.075 113.76) (end 215.265 113.76) (width 0.5) (layer "F.Cu") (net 10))
 (via (at 180.245 81.375) (size 0.8) (drill 0.4) (layers "F.Cu" "B.Cu") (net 10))
 (via (at 216.535 142.24) (size 0.8) (drill 0.4) (layers "F.Cu" "B.Cu") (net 10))
 (via (at 170.815 138.43) (size 0.8) (drill 0.4) (layers "F.Cu" "B.Cu") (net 10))
 (segment (start 218.44 144.145) (end 218.44 146.685) (width 0.5) (layer "B.Cu") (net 10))
 (segment (start 203.835 144.78) (end 202.565 143.51) (width 0.5) (layer "B.Cu") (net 10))
 (segment (start 177.165 142.215) (end 175.26 140.31) (width 0.5) (layer "B.Cu") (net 10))
 (segment (start 172.695 140.31) (end 170.815 138.43) (width 0.5) (layer "B.Cu") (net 10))
 (segment (start 205.105 147.955) (end 203.835 146.685) (width 0.5) (layer "B.Cu") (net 10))
 (segment (start 216.535 142.24) (end 218.44 144.145) (width 0.5) (layer "B.Cu") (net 10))
 (segment (start 177.165 142.24) (end 177.165 142.215) (width 0.5) (layer "B.Cu") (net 10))
 (segment (start 202.565 143.51) (end 178.435 143.51) (width 0.5) (layer "B.Cu") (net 10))
 (segment (start 175.26 140.31) (end 172.695 140.31) (width 0.5) (layer "B.Cu") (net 10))
 (segment (start 218.44 146.685) (end 217.17 147.955) (width 0.5) (layer "B.Cu") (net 10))
 (segment (start 217.17 147.955) (end 205.105 147.955) (width 0.5) (layer "B.Cu") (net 10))
 (segment (start 203.835 146.685) (end 203.835 144.78) (width 0.5) (layer "B.Cu") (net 10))
 (segment (start 180.245 81.375) (end 180.245 88.36) (width 0.5) (layer "B.Cu") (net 10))
 (segment (start 178.435 143.51) (end 177.165 142.24) (width 0.5) (layer "B.Cu") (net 10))
 (segment (start 215.265 97.79) (end 196.85 97.79) (width 0.5) (layer "F.Cu") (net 11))
 (segment (start 196.85 97.79) (end 195.58 99.06) (width 0.5) (layer "F.Cu") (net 11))
 (via (at 195.58 99.06) (size 0.8) (drill 0.4) (layers "F.Cu" "B.Cu") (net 11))
 (segment (start 193.135 101.505) (end 193.135 111.69) (width 0.5) (layer "B.Cu") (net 11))
 (segment (start 195.58 99.06) (end 193.135 101.505) (width 0.5) (layer "B.Cu") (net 11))
 (segment (start 199.39 147.32) (end 197.485 145.415) (width 0.25) (layer "F.Cu") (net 21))
 (segment (start 186.055 94.615) (end 186.69 93.98) (width 0.25) (layer "F.Cu") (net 21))
 (segment (start 186.055 114.935) (end 186.055 94.615) (width 0.25) (layer "F.Cu") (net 21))
 (segment (start 189.865 118.745) (end 186.055 114.935) (width 0.25) (layer "F.Cu") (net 21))
 (segment (start 206.375 142.24) (end 201.295 147.32) (width 0.25) (layer "F.Cu") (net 21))
 (segment (start 197.485 123.19) (end 193.04 118.745) (width 0.25) (layer "F.Cu") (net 21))
 (segment (start 193.04 118.745) (end 189.865 118.745) (width 0.25) (layer "F.Cu") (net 21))
 (segment (start 201.295 147.32) (end 199.39 147.32) (width 0.25) (layer "F.Cu") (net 21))
 (segment (start 197.485 145.415) (end 197.485 123.19) (width 0.25) (layer "F.Cu") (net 21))
 (via (at 186.69 93.98) (size 0.8) (drill 0.4) (layers "F.Cu" "B.Cu") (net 21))
 (via (at 197.485 123.19) (size 0.8) (drill 0.4) (layers "F.Cu" "B.Cu") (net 21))
 (segment (start 186.69 93.98) (end 193.675 93.98) (width 0.25) (layer "B.Cu") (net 21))
 (segment (start 198.145 122.53) (end 200.66 122.53) (width 0.25) (layer "B.Cu") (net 21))
 (segment (start 193.675 93.98) (end 195.485 92.17) (width 0.25) (layer "B.Cu") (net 21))
 (segment (start 197.485 123.19) (end 198.145 122.53) (width 0.25) (layer "B.Cu") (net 21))
 (segment (start 195.485 92.17) (end 195.485 88.36) (width 0.25) (layer "B.Cu") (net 21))
 (segment (start 180.975 54.61) (end 205.105 54.61) (width 0.25) (layer "F.Cu") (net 14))
 (segment (start 179.165 57.88) (end 179.165 56.42) (width 0.25) (layer "F.Cu") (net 14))
 (segment (start 207.01 71.12) (end 205.74 72.39) (width 0.25) (layer "F.Cu") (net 14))
 (segment (start 205.74 72.39) (end 204.47 72.39) (width 0.25) (layer "F.Cu") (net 14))
 (segment (start 207.01 56.515) (end 207.01 71.12) (width 0.25) (layer "F.Cu") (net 14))
 (segment (start 179.165 56.42) (end 180.975 54.61) (width 0.25) (layer "F.Cu") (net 14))
 (segment (start 205.105 54.61) (end 207.01 56.515) (width 0.25) (layer "F.Cu") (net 14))
 (via (at 204.47 72.39) (size 0.8) (drill 0.4) (layers "F.Cu" "B.Cu") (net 14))
 (segment (start 204.47 74.93) (end 205.105 75.565) (width 0.25) (layer "B.Cu") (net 14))
 (segment (start 198.755 100.33) (end 196.215 102.87) (width 0.25) (layer "B.Cu") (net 14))
 (segment (start 197.485 114.935) (end 197.51 114.91) (width 0.25) (layer "B.Cu") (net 14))
 (segment (start 197.51 114.91) (end 200.66 114.91) (width 0.25) (layer "B.Cu") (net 14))
 (segment (start 204.47 72.39) (end 204.47 74.93) (width 0.25) (layer "B.Cu") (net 14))
 (segment (start 196.215 102.87) (end 196.215 113.665) (width 0.25) (layer "B.Cu") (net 14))
 (segment (start 198.755 83.185) (end 198.755 100.33) (width 0.25) (layer "B.Cu") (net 14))
 (segment (start 205.105 75.565) (end 205.105 76.835) (width 0.25) (layer "B.Cu") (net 14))
 (segment (start 205.105 76.835) (end 198.755 83.185) (width 0.25) (layer "B.Cu") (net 14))
 (segment (start 196.215 113.665) (end 197.485 114.935) (width 0.25) (layer "B.Cu") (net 14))
 (segment (start 205.74 122.555) (end 203.835 122.555) (width 0.25) (layer "F.Cu") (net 12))
 (segment (start 211.995 116.3) (end 205.74 122.555) (width 0.25) (layer "F.Cu") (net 12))
 (segment (start 215.265 116.3) (end 211.995 116.3) (width 0.25) (layer "F.Cu") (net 12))
 (via (at 203.835 122.555) (size 0.8) (drill 0.4) (layers "F.Cu" "B.Cu") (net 12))
 (segment (start 203.175 122.555) (end 200.66 125.07) (width 0.25) (layer "B.Cu") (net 12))
 (segment (start 203.835 122.555) (end 203.175 122.555) (width 0.25) (layer "B.Cu") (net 12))
 (segment (start 204.47 55.245) (end 206.375 57.15) (width 0.25) (layer "F.Cu") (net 15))
 (segment (start 207.01 75.935) (end 204.735 75.935) (width 0.25) (layer "F.Cu") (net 15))
 (segment (start 191.77 55.245) (end 204.47 55.245) (width 0.25) (layer "F.Cu") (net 15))
 (segment (start 190.595 57.88) (end 190.595 56.42) (width 0.25) (layer "F.Cu") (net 15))
 (segment (start 206.375 69.215) (end 203.745 71.845) (width 0.25) (layer "F.Cu") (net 15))
 (segment (start 203.745 71.845) (end 203.745 74.84) (width 0.25) (layer "F.Cu") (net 15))
 (segment (start 204.735 75.935) (end 203.835 76.835) (width 0.25) (layer "F.Cu") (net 15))
 (segment (start 204.84 75.935) (end 207.01 75.935) (width 0.25) (layer "F.Cu") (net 15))
 (segment (start 190.595 56.42) (end 191.77 55.245) (width 0.25) (layer "F.Cu") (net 15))
 (segment (start 203.745 74.84) (end 204.84 75.935) (width 0.25) (layer "F.Cu") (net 15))
 (segment (start 206.375 57.15) (end 206.375 69.215) (width 0.25) (layer "F.Cu") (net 15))
 (via (at 203.835 76.835) (size 0.8) (drill 0.4) (layers "F.Cu" "B.Cu") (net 15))
 (segment (start 198.12 82.55) (end 198.12 99.695) (width 0.25) (layer "B.Cu") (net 15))
 (segment (start 195.58 122.53) (end 200.66 127.61) (width 0.25) (layer "B.Cu") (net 15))
 (segment (start 195.58 102.235) (end 195.58 122.53) (width 0.25) (layer "B.Cu") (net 15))
 (segment (start 203.835 76.835) (end 198.12 82.55) (width 0.25) (layer "B.Cu") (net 15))
 (segment (start 198.12 99.695) (end 195.58 102.235) (width 0.25) (layer "B.Cu") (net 15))
 (segment (start 197.485 93.98) (end 198.12 93.345) (width 0.25) (layer "F.Cu") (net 13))
 (segment (start 198.12 84.455) (end 201.64 80.935) (width 0.25) (layer "F.Cu") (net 13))
 (segment (start 193.675 97.79) (end 197.485 93.98) (width 0.25) (layer "F.Cu") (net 13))
 (segment (start 170.815 112.3) (end 170.815 108.585) (width 0.25) (layer "F.Cu") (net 13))
 (segment (start 198.12 93.345) (end 198.12 84.455) (width 0.25) (layer "F.Cu") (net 13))
 (segment (start 201.64 80.935) (end 207.01 80.935) (width 0.25) (layer "F.Cu") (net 13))
 (via (at 170.815 108.585) (size 0.8) (drill 0.4) (layers "F.Cu" "B.Cu") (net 13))
 (via (at 193.675 97.79) (size 0.8) (drill 0.4) (layers "F.Cu" "B.Cu") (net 13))
 (segment (start 175.26 101.6) (end 189.865 101.6) (width 0.25) (layer "B.Cu") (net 13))
 (segment (start 190.5 100.965) (end 193.675 97.79) (width 0.25) (layer "B.Cu") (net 13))
 (segment (start 172.72 106.68) (end 172.72 104.14) (width 0.25) (layer "B.Cu") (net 13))
 (segment (start 173.355 111.125) (end 173.355 115.57) (width 0.25) (layer "B.Cu") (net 13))
 (segment (start 173.38 115.57) (end 175.26 117.45) (width 0.25) (layer "B.Cu") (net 13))
 (segment (start 189.865 101.6) (end 190.5 100.965) (width 0.25) (layer "B.Cu") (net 13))
 (segment (start 170.815 108.585) (end 172.72 106.68) (width 0.25) (layer "B.Cu") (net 13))
 (segment (start 173.355 115.57) (end 173.38 115.57) (width 0.25) (layer "B.Cu") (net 13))
 (segment (start 172.72 104.14) (end 175.26 101.6) (width 0.25) (layer "B.Cu") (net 13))
 (segment (start 170.815 108.585) (end 173.355 111.125) (width 0.25) (layer "B.Cu") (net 13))
 (segment (start 200.025 86.36) (end 198.755 87.63) (width 0.25) (layer "F.Cu") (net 9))
 (segment (start 198.755 87.63) (end 198.755 93.98) (width 0.25) (layer "F.Cu") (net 9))
 (segment (start 198.755 93.98) (end 194.381755 98.353245) (width 0.25) (layer "F.Cu") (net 9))
 (segment (start 207.01 86.36) (end 200.025 86.36) (width 0.25) (layer "F.Cu") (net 9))
 (segment (start 194.381755 98.353245) (end 194.381755 98.496755) (width 0.25) (layer "F.Cu") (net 9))
 (via (at 194.381755 98.496755) (size 0.8) (drill 0.4) (layers "F.Cu" "B.Cu") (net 9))
 (segment (start 194.31 95.25) (end 173.99 95.25) (width 0.25) (layer "B.Cu") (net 9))
 (segment (start 170.815 98.425) (end 170.815 101.6) (width 0.25) (layer "B.Cu") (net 9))
 (segment (start 194.945 97.93351) (end 194.945 95.885) (width 0.25) (layer "B.Cu") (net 9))
 (segment (start 194.945 95.885) (end 194.31 95.25) (width 0.25) (layer "B.Cu") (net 9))
 (segment (start 194.381755 98.496755) (end 194.945 97.93351) (width 0.25) (layer "B.Cu") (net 9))
 (segment (start 173.99 95.25) (end 170.815 98.425) (width 0.25) (layer "B.Cu") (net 9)))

